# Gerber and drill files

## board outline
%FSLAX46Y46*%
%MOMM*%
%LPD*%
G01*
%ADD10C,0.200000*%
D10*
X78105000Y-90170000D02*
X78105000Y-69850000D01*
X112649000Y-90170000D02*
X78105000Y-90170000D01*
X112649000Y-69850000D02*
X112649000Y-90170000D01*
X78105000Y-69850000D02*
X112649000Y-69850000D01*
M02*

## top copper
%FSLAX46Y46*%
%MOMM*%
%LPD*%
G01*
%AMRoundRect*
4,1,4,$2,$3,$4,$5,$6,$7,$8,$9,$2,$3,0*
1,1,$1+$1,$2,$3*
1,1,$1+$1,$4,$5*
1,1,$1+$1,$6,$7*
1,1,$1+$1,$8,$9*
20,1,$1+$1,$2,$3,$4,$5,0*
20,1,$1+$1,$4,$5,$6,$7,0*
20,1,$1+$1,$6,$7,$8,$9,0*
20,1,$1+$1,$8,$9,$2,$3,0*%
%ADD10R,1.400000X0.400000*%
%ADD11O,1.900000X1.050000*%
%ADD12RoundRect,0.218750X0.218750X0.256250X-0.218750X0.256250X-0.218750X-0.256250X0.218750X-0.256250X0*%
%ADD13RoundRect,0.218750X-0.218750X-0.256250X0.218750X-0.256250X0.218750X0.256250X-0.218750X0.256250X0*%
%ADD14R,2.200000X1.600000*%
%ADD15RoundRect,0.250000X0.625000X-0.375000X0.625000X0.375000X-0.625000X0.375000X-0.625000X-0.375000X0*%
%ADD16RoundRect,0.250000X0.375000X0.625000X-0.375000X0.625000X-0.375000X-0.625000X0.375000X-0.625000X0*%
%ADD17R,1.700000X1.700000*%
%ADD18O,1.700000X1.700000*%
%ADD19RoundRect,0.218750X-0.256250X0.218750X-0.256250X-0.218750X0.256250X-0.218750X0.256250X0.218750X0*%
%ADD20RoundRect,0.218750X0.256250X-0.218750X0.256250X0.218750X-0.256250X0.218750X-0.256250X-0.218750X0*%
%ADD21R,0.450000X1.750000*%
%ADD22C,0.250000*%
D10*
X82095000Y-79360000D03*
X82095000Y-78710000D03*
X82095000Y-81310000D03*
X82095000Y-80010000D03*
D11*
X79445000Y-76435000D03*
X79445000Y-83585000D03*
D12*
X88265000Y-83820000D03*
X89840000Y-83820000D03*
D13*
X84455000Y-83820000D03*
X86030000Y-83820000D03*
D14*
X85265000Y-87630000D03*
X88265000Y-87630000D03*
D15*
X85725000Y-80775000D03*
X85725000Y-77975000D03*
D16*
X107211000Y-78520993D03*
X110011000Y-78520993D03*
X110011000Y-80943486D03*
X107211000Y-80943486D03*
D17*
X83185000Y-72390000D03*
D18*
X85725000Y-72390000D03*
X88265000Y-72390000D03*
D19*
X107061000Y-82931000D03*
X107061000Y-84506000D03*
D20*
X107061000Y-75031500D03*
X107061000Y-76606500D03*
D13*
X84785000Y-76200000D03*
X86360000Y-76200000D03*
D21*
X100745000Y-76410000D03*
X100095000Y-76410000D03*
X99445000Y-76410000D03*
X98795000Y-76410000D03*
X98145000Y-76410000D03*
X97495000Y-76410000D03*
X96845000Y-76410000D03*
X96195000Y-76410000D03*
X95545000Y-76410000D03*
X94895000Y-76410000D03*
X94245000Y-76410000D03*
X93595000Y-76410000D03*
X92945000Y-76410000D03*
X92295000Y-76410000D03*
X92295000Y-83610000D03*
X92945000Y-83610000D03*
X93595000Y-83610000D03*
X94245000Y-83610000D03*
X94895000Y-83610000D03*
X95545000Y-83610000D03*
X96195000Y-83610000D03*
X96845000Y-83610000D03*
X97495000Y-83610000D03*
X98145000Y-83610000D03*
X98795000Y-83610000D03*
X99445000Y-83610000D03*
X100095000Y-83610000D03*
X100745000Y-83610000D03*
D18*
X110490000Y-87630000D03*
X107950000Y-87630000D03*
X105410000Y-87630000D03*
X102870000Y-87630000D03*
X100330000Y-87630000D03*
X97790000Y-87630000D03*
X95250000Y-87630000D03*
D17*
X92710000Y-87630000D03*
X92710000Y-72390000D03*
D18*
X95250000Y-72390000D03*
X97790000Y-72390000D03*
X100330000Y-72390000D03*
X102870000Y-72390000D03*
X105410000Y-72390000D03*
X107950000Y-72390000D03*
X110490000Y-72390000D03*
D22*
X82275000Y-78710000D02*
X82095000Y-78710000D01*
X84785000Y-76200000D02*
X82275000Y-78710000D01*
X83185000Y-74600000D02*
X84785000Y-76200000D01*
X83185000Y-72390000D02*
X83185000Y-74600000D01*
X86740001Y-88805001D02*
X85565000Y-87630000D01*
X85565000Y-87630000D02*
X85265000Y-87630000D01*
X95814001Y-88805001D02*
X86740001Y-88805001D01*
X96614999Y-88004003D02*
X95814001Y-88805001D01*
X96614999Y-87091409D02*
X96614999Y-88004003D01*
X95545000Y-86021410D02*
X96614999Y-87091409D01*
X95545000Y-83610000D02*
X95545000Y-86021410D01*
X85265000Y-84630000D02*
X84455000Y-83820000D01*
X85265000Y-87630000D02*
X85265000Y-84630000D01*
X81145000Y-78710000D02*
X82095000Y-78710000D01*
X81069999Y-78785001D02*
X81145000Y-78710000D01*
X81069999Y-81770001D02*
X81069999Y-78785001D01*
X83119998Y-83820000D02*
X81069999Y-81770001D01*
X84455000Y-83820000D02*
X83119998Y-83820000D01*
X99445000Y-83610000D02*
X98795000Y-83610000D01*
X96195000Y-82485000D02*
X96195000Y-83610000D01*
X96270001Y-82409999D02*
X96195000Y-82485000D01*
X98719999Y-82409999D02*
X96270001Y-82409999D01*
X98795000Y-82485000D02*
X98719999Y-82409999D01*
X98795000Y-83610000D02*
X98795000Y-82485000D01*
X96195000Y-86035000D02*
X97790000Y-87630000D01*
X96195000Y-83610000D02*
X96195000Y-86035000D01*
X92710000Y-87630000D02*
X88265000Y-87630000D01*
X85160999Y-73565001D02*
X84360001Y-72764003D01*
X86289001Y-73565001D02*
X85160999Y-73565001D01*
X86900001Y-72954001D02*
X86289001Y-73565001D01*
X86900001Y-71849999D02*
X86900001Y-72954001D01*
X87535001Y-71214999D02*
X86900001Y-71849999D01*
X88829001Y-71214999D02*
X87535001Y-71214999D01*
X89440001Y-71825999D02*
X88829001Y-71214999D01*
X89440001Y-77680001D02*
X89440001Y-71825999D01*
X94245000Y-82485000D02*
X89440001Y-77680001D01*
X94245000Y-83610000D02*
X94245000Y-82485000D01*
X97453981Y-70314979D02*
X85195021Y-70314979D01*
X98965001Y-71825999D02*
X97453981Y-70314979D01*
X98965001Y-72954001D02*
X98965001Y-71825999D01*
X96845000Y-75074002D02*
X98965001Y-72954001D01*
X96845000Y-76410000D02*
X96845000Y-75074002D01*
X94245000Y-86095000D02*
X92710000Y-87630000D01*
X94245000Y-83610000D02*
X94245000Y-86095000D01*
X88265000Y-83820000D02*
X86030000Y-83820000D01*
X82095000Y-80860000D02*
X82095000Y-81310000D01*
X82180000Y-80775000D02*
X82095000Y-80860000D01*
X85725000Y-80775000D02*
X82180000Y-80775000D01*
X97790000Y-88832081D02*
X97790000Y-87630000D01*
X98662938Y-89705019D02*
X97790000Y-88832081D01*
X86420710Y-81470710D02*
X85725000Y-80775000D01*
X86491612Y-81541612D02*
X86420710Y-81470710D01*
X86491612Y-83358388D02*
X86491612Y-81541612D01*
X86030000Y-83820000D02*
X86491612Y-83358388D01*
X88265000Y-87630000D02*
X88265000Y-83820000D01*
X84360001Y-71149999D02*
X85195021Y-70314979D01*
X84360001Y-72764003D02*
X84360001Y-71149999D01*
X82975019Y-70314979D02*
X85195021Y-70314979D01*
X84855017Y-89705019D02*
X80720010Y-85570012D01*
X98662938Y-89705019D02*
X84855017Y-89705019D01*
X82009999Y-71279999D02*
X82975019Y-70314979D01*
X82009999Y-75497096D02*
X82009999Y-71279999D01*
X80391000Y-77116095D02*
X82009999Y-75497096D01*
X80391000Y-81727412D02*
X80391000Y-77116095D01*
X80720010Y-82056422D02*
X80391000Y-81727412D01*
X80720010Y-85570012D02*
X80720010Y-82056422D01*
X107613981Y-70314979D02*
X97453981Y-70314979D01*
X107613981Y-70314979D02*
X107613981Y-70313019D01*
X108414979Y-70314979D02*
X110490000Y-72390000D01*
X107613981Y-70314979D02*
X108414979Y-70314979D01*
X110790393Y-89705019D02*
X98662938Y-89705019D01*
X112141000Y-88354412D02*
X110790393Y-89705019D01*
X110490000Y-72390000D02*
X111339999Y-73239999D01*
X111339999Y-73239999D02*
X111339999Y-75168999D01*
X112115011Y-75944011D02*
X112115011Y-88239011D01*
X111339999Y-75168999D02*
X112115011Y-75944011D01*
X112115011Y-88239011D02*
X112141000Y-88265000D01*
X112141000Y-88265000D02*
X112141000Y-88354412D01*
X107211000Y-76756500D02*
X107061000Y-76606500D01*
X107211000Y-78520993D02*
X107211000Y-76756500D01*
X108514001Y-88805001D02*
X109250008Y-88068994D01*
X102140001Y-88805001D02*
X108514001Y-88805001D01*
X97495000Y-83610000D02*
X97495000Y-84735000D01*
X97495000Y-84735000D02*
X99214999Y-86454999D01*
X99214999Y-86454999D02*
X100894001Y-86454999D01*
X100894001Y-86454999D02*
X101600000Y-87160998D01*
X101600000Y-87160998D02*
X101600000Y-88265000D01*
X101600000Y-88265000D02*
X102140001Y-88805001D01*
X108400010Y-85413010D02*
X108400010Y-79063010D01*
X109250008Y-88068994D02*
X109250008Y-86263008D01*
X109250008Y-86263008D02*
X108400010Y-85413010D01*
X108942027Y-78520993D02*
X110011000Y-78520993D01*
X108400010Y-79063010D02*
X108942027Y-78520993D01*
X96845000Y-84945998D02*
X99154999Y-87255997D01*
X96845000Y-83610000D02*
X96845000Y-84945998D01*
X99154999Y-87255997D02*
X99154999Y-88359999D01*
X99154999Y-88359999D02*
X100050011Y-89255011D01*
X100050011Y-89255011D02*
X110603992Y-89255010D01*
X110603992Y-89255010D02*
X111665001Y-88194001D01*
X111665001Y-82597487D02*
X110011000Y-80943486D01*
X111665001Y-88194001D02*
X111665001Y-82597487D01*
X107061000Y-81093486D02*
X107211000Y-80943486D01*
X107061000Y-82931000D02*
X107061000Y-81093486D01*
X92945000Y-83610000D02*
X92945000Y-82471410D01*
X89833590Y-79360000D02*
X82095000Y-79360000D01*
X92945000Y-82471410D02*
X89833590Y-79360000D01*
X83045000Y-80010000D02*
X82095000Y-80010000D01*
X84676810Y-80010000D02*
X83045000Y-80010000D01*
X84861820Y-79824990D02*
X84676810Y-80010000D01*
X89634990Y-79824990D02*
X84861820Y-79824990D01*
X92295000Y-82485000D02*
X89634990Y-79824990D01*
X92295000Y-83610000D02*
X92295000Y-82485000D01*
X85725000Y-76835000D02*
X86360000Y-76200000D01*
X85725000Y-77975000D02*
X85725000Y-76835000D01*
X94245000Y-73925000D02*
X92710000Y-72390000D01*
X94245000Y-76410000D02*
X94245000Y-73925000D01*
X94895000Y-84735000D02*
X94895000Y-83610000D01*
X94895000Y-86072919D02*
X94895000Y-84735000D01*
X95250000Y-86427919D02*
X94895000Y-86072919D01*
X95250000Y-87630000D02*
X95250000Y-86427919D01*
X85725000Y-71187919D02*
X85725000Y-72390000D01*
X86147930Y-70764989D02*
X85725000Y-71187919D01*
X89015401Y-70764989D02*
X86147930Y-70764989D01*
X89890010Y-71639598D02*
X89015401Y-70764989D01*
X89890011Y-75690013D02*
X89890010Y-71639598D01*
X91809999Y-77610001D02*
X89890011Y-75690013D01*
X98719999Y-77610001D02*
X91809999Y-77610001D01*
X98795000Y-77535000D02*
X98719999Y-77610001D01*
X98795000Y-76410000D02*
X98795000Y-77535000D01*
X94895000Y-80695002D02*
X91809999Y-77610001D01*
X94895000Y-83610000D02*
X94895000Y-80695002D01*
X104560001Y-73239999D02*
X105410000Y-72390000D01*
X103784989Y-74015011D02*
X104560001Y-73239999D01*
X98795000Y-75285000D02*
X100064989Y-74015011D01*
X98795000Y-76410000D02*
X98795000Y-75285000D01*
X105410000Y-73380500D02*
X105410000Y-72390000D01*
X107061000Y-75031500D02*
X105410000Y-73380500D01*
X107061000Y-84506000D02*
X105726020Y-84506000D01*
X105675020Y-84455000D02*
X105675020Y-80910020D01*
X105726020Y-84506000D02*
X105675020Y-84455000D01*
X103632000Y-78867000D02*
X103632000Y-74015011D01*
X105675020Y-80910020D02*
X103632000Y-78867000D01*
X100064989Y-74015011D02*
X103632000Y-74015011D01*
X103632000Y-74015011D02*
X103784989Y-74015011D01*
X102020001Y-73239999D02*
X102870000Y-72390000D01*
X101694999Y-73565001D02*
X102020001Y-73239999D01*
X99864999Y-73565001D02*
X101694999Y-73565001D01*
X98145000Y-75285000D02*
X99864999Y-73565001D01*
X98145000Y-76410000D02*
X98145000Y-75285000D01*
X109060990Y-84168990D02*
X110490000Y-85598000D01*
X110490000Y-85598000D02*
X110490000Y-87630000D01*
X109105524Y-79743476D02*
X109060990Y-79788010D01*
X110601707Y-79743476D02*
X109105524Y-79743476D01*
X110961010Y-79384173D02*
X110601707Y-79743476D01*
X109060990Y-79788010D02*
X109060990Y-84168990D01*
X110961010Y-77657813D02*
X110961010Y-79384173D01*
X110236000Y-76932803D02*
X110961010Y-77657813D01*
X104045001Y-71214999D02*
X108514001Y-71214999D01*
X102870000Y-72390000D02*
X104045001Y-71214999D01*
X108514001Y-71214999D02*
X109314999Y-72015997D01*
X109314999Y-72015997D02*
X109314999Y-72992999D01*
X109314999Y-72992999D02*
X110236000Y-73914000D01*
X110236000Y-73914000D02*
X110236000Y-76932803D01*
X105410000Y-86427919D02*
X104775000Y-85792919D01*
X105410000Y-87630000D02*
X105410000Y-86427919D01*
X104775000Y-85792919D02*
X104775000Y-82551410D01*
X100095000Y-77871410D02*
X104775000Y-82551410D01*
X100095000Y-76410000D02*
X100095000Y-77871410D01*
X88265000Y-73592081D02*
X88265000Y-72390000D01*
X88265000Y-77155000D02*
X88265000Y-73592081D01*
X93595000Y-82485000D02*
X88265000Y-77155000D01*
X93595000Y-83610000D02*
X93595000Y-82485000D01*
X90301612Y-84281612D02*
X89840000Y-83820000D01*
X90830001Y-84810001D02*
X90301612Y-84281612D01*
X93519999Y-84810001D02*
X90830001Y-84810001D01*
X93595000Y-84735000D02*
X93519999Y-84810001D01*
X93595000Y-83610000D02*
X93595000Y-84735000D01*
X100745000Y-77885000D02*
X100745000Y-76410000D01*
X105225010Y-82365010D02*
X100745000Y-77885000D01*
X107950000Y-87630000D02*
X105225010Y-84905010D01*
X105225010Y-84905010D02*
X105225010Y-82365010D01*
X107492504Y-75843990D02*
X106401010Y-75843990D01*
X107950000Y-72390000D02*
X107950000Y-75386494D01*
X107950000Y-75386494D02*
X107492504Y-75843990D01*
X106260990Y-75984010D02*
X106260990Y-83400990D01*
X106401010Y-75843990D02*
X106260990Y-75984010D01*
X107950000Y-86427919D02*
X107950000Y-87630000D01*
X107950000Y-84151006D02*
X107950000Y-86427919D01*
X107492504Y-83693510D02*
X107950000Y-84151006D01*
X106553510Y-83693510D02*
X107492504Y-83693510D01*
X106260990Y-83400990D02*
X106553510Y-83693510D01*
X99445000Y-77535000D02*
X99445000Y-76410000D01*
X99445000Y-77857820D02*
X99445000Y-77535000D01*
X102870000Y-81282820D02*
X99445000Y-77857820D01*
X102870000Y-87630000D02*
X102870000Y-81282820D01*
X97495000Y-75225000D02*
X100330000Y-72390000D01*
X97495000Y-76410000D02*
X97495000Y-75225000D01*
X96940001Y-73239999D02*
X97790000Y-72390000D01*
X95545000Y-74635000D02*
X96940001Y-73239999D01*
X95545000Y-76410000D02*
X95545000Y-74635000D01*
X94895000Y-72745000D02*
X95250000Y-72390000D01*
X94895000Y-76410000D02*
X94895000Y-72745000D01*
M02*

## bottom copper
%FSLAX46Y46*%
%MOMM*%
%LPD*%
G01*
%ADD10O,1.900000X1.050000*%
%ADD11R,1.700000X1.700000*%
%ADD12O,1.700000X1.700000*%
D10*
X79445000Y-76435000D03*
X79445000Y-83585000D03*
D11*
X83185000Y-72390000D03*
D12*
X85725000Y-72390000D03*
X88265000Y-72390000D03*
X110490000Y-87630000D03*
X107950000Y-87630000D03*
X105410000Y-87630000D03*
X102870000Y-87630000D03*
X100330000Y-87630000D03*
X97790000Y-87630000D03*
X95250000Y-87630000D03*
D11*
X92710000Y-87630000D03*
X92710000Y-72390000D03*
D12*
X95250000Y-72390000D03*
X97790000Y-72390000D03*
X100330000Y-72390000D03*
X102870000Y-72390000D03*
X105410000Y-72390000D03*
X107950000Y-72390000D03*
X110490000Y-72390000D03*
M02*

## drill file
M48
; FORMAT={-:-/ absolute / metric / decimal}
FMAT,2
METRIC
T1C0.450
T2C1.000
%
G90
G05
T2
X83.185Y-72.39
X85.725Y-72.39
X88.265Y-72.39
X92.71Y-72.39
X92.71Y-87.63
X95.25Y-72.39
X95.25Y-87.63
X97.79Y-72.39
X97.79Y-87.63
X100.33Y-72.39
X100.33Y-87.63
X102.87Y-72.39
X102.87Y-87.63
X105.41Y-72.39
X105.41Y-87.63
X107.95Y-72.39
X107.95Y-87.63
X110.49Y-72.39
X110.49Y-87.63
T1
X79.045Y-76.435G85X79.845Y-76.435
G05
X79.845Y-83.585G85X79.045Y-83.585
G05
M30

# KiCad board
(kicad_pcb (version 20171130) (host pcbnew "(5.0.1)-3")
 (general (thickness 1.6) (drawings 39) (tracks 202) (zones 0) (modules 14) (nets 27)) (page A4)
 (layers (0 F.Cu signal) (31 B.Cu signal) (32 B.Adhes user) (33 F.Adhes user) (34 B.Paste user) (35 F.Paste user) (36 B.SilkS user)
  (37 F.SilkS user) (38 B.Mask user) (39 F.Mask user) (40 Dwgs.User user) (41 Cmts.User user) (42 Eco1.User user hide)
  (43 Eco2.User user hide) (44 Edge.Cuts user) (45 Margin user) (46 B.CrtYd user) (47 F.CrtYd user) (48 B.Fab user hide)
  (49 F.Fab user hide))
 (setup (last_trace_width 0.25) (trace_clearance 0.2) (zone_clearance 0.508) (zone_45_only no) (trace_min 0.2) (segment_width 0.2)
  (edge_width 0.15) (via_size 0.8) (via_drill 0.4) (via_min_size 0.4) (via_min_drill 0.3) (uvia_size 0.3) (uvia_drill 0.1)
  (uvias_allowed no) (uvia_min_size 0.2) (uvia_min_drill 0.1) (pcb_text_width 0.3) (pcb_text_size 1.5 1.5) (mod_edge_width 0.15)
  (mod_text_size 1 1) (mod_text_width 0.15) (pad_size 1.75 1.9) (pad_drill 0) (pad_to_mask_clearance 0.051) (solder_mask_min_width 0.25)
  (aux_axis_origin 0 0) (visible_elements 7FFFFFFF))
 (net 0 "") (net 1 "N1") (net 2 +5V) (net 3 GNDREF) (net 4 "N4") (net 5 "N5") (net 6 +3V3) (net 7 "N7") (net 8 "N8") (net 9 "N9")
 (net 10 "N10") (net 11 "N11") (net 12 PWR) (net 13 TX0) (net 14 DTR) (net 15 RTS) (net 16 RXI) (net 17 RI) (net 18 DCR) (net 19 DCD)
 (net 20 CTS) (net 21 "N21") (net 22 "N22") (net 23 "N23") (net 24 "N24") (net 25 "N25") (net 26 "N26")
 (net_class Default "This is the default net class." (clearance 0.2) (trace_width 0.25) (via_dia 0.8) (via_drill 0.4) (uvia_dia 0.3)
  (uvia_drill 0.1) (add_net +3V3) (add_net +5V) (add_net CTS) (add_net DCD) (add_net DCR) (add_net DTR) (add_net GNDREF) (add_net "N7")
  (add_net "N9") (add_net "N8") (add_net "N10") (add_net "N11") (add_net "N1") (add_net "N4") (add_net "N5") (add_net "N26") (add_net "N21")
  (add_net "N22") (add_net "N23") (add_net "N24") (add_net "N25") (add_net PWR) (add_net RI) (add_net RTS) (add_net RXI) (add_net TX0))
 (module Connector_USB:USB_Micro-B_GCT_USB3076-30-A (layer F.Cu) (at 80.645 80.01 270)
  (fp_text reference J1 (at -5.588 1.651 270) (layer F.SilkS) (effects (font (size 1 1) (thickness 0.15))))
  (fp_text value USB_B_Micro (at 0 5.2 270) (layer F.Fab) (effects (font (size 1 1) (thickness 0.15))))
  (pad 2 smd rect (at -0.65 -1.45 270) (size 0.4 1.4) (layers F.Cu F.Paste F.Mask) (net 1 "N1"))
  (pad 1 smd rect (at -1.3 -1.45 270) (size 0.4 1.4) (layers F.Cu F.Paste F.Mask) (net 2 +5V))
  (pad 5 smd rect (at 1.3 -1.45 270) (size 0.4 1.4) (layers F.Cu F.Paste F.Mask) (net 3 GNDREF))
  (pad 3 smd rect (at 0 -1.45 270) (size 0.4 1.4) (layers F.Cu F.Paste F.Mask) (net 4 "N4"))
  (pad 6 thru_hole oval (at -3.575 1.2 90) (size 1.05 1.9) (drill oval 0.45 1.25) (layers *.Cu *.Mask) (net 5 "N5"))
  (pad 6 thru_hole oval (at 3.575 1.2 270) (size 1.05 1.9) (drill oval 0.45 1.25) (layers *.Cu *.Mask) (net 5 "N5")))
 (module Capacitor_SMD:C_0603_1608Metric (layer F.Cu) (at 89.0525 83.82 180)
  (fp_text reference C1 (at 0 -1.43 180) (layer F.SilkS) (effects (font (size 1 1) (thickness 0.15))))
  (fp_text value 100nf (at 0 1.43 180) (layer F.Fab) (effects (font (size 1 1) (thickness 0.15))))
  (pad 2 smd roundrect (at 0.7875 0 180) (size 0.875 0.95) (layers F.Cu F.Paste F.Mask) (roundrect_rratio 0.25) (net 3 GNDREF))
  (pad 1 smd roundrect (at -0.7875 0 180) (size 0.875 0.95) (layers F.Cu F.Paste F.Mask) (roundrect_rratio 0.25) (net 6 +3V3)))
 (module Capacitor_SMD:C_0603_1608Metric (layer F.Cu) (at 85.2425 83.82)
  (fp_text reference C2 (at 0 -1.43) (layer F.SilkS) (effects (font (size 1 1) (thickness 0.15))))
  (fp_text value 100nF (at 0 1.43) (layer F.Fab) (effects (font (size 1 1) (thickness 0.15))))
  (pad 1 smd roundrect (at -0.7875 0) (size 0.875 0.95) (layers F.Cu F.Paste F.Mask) (roundrect_rratio 0.25) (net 2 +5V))
  (pad 2 smd roundrect (at 0.7875 0) (size 0.875 0.95) (layers F.Cu F.Paste F.Mask) (roundrect_rratio 0.25) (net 3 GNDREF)))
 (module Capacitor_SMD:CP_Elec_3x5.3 (layer F.Cu) (at 86.765 87.63)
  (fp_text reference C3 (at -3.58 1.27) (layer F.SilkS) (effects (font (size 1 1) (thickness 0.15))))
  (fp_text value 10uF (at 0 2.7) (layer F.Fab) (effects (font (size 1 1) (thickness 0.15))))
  (pad 1 smd rect (at -1.5 0) (size 2.2 1.6) (layers F.Cu F.Paste F.Mask) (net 2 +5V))
  (pad 2 smd rect (at 1.5 0) (size 2.2 1.6) (layers F.Cu F.Paste F.Mask) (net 3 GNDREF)))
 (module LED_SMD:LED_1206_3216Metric (layer F.Cu) (at 85.725 79.375 90)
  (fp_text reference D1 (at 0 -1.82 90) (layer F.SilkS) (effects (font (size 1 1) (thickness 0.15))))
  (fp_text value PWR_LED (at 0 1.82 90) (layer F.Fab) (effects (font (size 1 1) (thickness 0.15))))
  (pad 1 smd roundrect (at -1.4 0 90) (size 1.25 1.75) (layers F.Cu F.Paste F.Mask) (roundrect_rratio 0.2) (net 3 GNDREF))
  (pad 2 smd roundrect (at 1.4 0 90) (size 1.25 1.75) (layers F.Cu F.Paste F.Mask) (roundrect_rratio 0.2) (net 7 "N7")))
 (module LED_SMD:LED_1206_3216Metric (layer F.Cu) (at 108.611 78.520993 180)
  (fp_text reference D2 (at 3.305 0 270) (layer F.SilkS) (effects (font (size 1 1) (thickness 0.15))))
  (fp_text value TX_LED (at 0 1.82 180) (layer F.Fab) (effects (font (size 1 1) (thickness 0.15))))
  (pad 2 smd roundrect (at 1.4 0 180) (size 1.25 1.75) (layers F.Cu F.Paste F.Mask) (roundrect_rratio 0.2) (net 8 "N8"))
  (pad 1 smd roundrect (at -1.4 0 180) (size 1.25 1.75) (layers F.Cu F.Paste F.Mask) (roundrect_rratio 0.2) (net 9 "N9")))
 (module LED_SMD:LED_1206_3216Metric (layer F.Cu) (at 108.611 80.943486 180)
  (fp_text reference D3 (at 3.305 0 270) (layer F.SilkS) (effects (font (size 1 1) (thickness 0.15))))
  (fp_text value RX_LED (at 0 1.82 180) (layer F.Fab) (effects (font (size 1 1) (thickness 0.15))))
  (pad 1 smd roundrect (at -1.4 0 180) (size 1.25 1.75) (layers F.Cu F.Paste F.Mask) (roundrect_rratio 0.2) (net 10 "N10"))
  (pad 2 smd roundrect (at 1.4 0 180) (size 1.25 1.75) (layers F.Cu F.Paste F.Mask) (roundrect_rratio 0.2) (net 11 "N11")))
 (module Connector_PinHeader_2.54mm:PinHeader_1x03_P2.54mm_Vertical (layer F.Cu) (at 83.185 72.39 90)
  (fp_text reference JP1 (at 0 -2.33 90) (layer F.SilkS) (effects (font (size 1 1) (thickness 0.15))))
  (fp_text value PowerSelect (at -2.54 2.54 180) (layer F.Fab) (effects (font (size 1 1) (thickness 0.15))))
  (pad 1 thru_hole rect (at 0 0 90) (size 1.7 1.7) (drill 1) (layers *.Cu *.Mask) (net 2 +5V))
  (pad 2 thru_hole oval (at 0 2.54 90) (size 1.7 1.7) (drill 1) (layers *.Cu *.Mask) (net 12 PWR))
  (pad 3 thru_hole oval (at 0 5.08 90) (size 1.7 1.7) (drill 1) (layers *.Cu *.Mask) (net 6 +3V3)))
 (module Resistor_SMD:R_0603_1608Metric (layer F.Cu) (at 107.061 83.7185 270)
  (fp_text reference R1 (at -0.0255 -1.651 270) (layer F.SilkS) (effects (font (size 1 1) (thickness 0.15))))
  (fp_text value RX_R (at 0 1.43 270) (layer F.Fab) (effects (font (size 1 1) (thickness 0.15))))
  (pad 1 smd roundrect (at -0.7875 0 270) (size 0.875 0.95) (layers F.Cu F.Paste F.Mask) (roundrect_rratio 0.25) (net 11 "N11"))
  (pad 2 smd roundrect (at 0.7875 0 270) (size 0.875 0.95) (layers F.Cu F.Paste F.Mask) (roundrect_rratio 0.25) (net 12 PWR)))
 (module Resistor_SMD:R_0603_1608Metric (layer F.Cu) (at 107.061 75.819 90)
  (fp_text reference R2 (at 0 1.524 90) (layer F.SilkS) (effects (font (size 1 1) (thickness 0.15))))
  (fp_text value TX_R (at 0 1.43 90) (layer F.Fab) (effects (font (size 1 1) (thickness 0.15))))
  (pad 2 smd roundrect (at 0.7875 0 90) (size 0.875 0.95) (layers F.Cu F.Paste F.Mask) (roundrect_rratio 0.25) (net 12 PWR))
  (pad 1 smd roundrect (at -0.7875 0 90) (size 0.875 0.95) (layers F.Cu F.Paste F.Mask) (roundrect_rratio 0.25) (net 8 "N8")))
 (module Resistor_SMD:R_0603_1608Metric (layer F.Cu) (at 85.5725 76.2)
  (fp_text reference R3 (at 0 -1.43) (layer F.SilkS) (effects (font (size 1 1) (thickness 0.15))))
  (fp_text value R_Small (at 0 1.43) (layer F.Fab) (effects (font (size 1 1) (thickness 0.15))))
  (pad 1 smd roundrect (at -0.7875 0) (size 0.875 0.95) (layers F.Cu F.Paste F.Mask) (roundrect_rratio 0.25) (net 2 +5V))
  (pad 2 smd roundrect (at 0.7875 0) (size 0.875 0.95) (layers F.Cu F.Paste F.Mask) (roundrect_rratio 0.25) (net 7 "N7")))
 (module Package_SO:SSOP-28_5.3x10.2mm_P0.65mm (layer F.Cu) (at 96.52 80.01 270)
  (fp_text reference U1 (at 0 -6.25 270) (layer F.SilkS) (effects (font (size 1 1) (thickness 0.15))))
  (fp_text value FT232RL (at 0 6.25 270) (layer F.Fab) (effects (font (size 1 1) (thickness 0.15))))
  (pad 1 smd rect (at -3.6 -4.225 270) (size 1.75 0.45) (layers F.Cu F.Paste F.Mask) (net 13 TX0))
  (pad 2 smd rect (at -3.6 -3.575 270) (size 1.75 0.45) (layers F.Cu F.Paste F.Mask) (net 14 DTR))
  (pad 3 smd rect (at -3.6 -2.925 270) (size 1.75 0.45) (layers F.Cu F.Paste F.Mask) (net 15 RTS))
  (pad 4 smd rect (at -3.6 -2.275 270) (size 1.75 0.45) (layers F.Cu F.Paste F.Mask) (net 12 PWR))
  (pad 5 smd rect (at -3.6 -1.625 270) (size 1.75 0.45) (layers F.Cu F.Paste F.Mask) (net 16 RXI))
  (pad 6 smd rect (at -3.6 -0.975 270) (size 1.75 0.45) (layers F.Cu F.Paste F.Mask) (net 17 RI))
  (pad 7 smd rect (at -3.6 -0.325 270) (size 1.75 0.45) (layers F.Cu F.Paste F.Mask) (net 3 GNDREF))
  (pad 8 smd rect (at -3.6 0.325 270) (size 1.75 0.45) (layers F.Cu F.Paste F.Mask))
  (pad 9 smd rect (at -3.6 0.975 270) (size 1.75 0.45) (layers F.Cu F.Paste F.Mask) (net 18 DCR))
  (pad 10 smd rect (at -3.6 1.625 270) (size 1.75 0.45) (layers F.Cu F.Paste F.Mask) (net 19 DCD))
  (pad 11 smd rect (at -3.6 2.275 270) (size 1.75 0.45) (layers F.Cu F.Paste F.Mask) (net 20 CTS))
  (pad 12 smd rect (at -3.6 2.925 270) (size 1.75 0.45) (layers F.Cu F.Paste F.Mask) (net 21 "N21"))
  (pad 13 smd rect (at -3.6 3.575 270) (size 1.75 0.45) (layers F.Cu F.Paste F.Mask) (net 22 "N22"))
  (pad 14 smd rect (at -3.6 4.225 270) (size 1.75 0.45) (layers F.Cu F.Paste F.Mask) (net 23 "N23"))
  (pad 15 smd rect (at 3.6 4.225 270) (size 1.75 0.45) (layers F.Cu F.Paste F.Mask) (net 4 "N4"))
  (pad 16 smd rect (at 3.6 3.575 270) (size 1.75 0.45) (layers F.Cu F.Paste F.Mask) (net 1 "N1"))
  (pad 17 smd rect (at 3.6 2.925 270) (size 1.75 0.45) (layers F.Cu F.Paste F.Mask) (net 6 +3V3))
  (pad 18 smd rect (at 3.6 2.275 270) (size 1.75 0.45) (layers F.Cu F.Paste F.Mask) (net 3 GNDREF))
  (pad 19 smd rect (at 3.6 1.625 270) (size 1.75 0.45) (layers F.Cu F.Paste F.Mask) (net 12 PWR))
  (pad 20 smd rect (at 3.6 0.975 270) (size 1.75 0.45) (layers F.Cu F.Paste F.Mask) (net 2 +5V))
  (pad 21 smd rect (at 3.6 0.325 270) (size 1.75 0.45) (layers F.Cu F.Paste F.Mask) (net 3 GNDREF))
  (pad 22 smd rect (at 3.6 -0.325 270) (size 1.75 0.45) (layers F.Cu F.Paste F.Mask) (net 10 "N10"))
  (pad 23 smd rect (at 3.6 -0.975 270) (size 1.75 0.45) (layers F.Cu F.Paste F.Mask) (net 9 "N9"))
  (pad 24 smd rect (at 3.6 -1.625 270) (size 1.75 0.45) (layers F.Cu F.Paste F.Mask))
  (pad 25 smd rect (at 3.6 -2.275 270) (size 1.75 0.45) (layers F.Cu F.Paste F.Mask) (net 3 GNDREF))
  (pad 26 smd rect (at 3.6 -2.925 270) (size 1.75 0.45) (layers F.Cu F.Paste F.Mask) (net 3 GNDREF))
  (pad 27 smd rect (at 3.6 -3.575 270) (size 1.75 0.45) (layers F.Cu F.Paste F.Mask) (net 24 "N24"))
  (pad 28 smd rect (at 3.6 -4.225 270) (size 1.75 0.45) (layers F.Cu F.Paste F.Mask) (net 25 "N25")))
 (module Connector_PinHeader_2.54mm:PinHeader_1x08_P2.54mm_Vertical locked (layer F.Cu) (at 92.71 87.63 90)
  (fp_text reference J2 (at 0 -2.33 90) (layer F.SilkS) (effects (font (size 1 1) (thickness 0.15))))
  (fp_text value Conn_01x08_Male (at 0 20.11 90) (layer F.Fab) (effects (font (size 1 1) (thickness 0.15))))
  (pad 8 thru_hole oval (at 0 17.78 90) (size 1.7 1.7) (drill 1) (layers *.Cu *.Mask) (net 16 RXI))
  (pad 7 thru_hole oval (at 0 15.24 90) (size 1.7 1.7) (drill 1) (layers *.Cu *.Mask) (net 13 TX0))
  (pad 6 thru_hole oval (at 0 12.7 90) (size 1.7 1.7) (drill 1) (layers *.Cu *.Mask) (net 14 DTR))
  (pad 5 thru_hole oval (at 0 10.16 90) (size 1.7 1.7) (drill 1) (layers *.Cu *.Mask) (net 15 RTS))
  (pad 4 thru_hole oval (at 0 7.62 90) (size 1.7 1.7) (drill 1) (layers *.Cu *.Mask) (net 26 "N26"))
  (pad 3 thru_hole oval (at 0 5.08 90) (size 1.7 1.7) (drill 1) (layers *.Cu *.Mask) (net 3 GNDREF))
  (pad 2 thru_hole oval (at 0 2.54 90) (size 1.7 1.7) (drill 1) (layers *.Cu *.Mask) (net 12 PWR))
  (pad 1 thru_hole rect (at 0 0 90) (size 1.7 1.7) (drill 1) (layers *.Cu *.Mask) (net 3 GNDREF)))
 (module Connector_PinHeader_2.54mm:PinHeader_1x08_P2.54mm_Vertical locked (layer F.Cu) (at 92.71 72.39 90)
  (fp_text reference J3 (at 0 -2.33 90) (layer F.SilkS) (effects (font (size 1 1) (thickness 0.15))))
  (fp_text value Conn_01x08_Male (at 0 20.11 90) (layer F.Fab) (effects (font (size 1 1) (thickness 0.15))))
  (pad 1 thru_hole rect (at 0 0 90) (size 1.7 1.7) (drill 1) (layers *.Cu *.Mask) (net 20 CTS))
  (pad 2 thru_hole oval (at 0 2.54 90) (size 1.7 1.7) (drill 1) (layers *.Cu *.Mask) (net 19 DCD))
  (pad 3 thru_hole oval (at 0 5.08 90) (size 1.7 1.7) (drill 1) (layers *.Cu *.Mask) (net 18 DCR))
  (pad 4 thru_hole oval (at 0 7.62 90) (size 1.7 1.7) (drill 1) (layers *.Cu *.Mask) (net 17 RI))
  (pad 5 thru_hole oval (at 0 10.16 90) (size 1.7 1.7) (drill 1) (layers *.Cu *.Mask) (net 16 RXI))
  (pad 6 thru_hole oval (at 0 12.7 90) (size 1.7 1.7) (drill 1) (layers *.Cu *.Mask) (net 12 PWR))
  (pad 7 thru_hole oval (at 0 15.24 90) (size 1.7 1.7) (drill 1) (layers *.Cu *.Mask) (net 13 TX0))
  (pad 8 thru_hole oval (at 0 17.78 90) (size 1.7 1.7) (drill 1) (layers *.Cu *.Mask) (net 3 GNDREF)))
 (gr_line (start 78.105 90.17) (end 78.105 69.85) (layer Edge.Cuts) (width 0.2))
 (gr_line (start 112.649 90.17) (end 78.105 90.17) (layer Edge.Cuts) (width 0.2))
 (gr_line (start 112.649 69.85) (end 112.649 90.17) (layer Edge.Cuts) (width 0.2))
 (gr_line (start 78.105 69.85) (end 112.649 69.85) (layer Edge.Cuts) (width 0.2))
 (segment (start 82.275 78.71) (end 82.095 78.71) (width 0.25) (layer F.Cu) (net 2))
 (segment (start 84.785 76.2) (end 82.275 78.71) (width 0.25) (layer F.Cu) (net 2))
 (segment (start 83.185 74.6) (end 84.785 76.2) (width 0.25) (layer F.Cu) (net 2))
 (segment (start 83.185 72.39) (end 83.185 74.6) (width 0.25) (layer F.Cu) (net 2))
 (segment (start 86.740001 88.805001) (end 85.565 87.63) (width 0.25) (layer F.Cu) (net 2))
 (segment (start 85.565 87.63) (end 85.265 87.63) (width 0.25) (layer F.Cu) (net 2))
 (segment (start 95.814001 88.805001) (end 86.740001 88.805001) (width 0.25) (layer F.Cu) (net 2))
 (segment (start 96.614999 88.004003) (end 95.814001 88.805001) (width 0.25) (layer F.Cu) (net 2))
 (segment (start 96.614999 87.091409) (end 96.614999 88.004003) (width 0.25) (layer F.Cu) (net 2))
 (segment (start 95.545 86.02141) (end 96.614999 87.091409) (width 0.25) (layer F.Cu) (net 2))
 (segment (start 95.545 83.61) (end 95.545 86.02141) (width 0.25) (layer F.Cu) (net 2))
 (segment (start 85.265 84.63) (end 84.455 83.82) (width 0.25) (layer F.Cu) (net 2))
 (segment (start 85.265 87.63) (end 85.265 84.63) (width 0.25) (layer F.Cu) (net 2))
 (segment (start 81.145 78.71) (end 82.095 78.71) (width 0.25) (layer F.Cu) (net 2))
 (segment (start 81.069999 78.785001) (end 81.145 78.71) (width 0.25) (layer F.Cu) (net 2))
 (segment (start 81.069999 81.770001) (end 81.069999 78.785001) (width 0.25) (layer F.Cu) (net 2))
 (segment (start 83.119998 83.82) (end 81.069999 81.770001) (width 0.25) (layer F.Cu) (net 2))
 (segment (start 84.455 83.82) (end 83.119998 83.82) (width 0.25) (layer F.Cu) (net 2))
 (segment (start 99.445 83.61) (end 98.795 83.61) (width 0.25) (layer F.Cu) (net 3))
 (segment (start 96.195 82.485) (end 96.195 83.61) (width 0.25) (layer F.Cu) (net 3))
 (segment (start 96.270001 82.409999) (end 96.195 82.485) (width 0.25) (layer F.Cu) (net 3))
 (segment (start 98.719999 82.409999) (end 96.270001 82.409999) (width 0.25) (layer F.Cu) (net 3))
 (segment (start 98.795 82.485) (end 98.719999 82.409999) (width 0.25) (layer F.Cu) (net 3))
 (segment (start 98.795 83.61) (end 98.795 82.485) (width 0.25) (layer F.Cu) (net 3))
 (segment (start 96.195 86.035) (end 97.79 87.63) (width 0.25) (layer F.Cu) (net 3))
 (segment (start 96.195 83.61) (end 96.195 86.035) (width 0.25) (layer F.Cu) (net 3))
 (segment (start 92.71 87.63) (end 88.265 87.63) (width 0.25) (layer F.Cu) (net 3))
 (segment (start 85.160999 73.565001) (end 84.360001 72.764003) (width 0.25) (layer F.Cu) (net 3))
 (segment (start 86.289001 73.565001) (end 85.160999 73.565001) (width 0.25) (layer F.Cu) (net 3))
 (segment (start 86.900001 72.954001) (end 86.289001 73.565001) (width 0.25) (layer F.Cu) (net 3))
 (segment (start 86.900001 71.849999) (end 86.900001 72.954001) (width 0.25) (layer F.Cu) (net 3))
 (segment (start 87.535001 71.214999) (end 86.900001 71.849999) (width 0.25) (layer F.Cu) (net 3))
 (segment (start 88.829001 71.214999) (end 87.535001 71.214999) (width 0.25) (layer F.Cu) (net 3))
 (segment (start 89.440001 71.825999) (end 88.829001 71.214999) (width 0.25) (layer F.Cu) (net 3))
 (segment (start 89.440001 77.680001) (end 89.440001 71.825999) (width 0.25) (layer F.Cu) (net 3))
 (segment (start 94.245 82.485) (end 89.440001 77.680001) (width 0.25) (layer F.Cu) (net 3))
 (segment (start 94.245 83.61) (end 94.245 82.485) (width 0.25) (layer F.Cu) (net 3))
 (segment (start 97.453981 70.314979) (end 85.195021 70.314979) (width 0.25) (layer F.Cu) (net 3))
 (segment (start 98.965001 71.825999) (end 97.453981 70.314979) (width 0.25) (layer F.Cu) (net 3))
 (segment (start 98.965001 72.954001) (end 98.965001 71.825999) (width 0.25) (layer F.Cu) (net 3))
 (segment (start 96.845 75.074002) (end 98.965001 72.954001) (width 0.25) (layer F.Cu) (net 3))
 (segment (start 96.845 76.41) (end 96.845 75.074002) (width 0.25) (layer F.Cu) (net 3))
 (segment (start 94.245 86.095) (end 92.71 87.63) (width 0.25) (layer F.Cu) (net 3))
 (segment (start 94.245 83.61) (end 94.245 86.095) (width 0.25) (layer F.Cu) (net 3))
 (segment (start 88.265 83.82) (end 86.03 83.82) (width 0.25) (layer F.Cu) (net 3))
 (segment (start 82.095 80.86) (end 82.095 81.31) (width 0.25) (layer F.Cu) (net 3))
 (segment (start 82.18 80.775) (end 82.095 80.86) (width 0.25) (layer F.Cu) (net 3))
 (segment (start 85.725 80.775) (end 82.18 80.775) (width 0.25) (layer F.Cu) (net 3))
 (segment (start 97.79 88.832081) (end 97.79 87.63) (width 0.25) (layer F.Cu) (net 3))
 (segment (start 98.662938 89.705019) (end 97.79 88.832081) (width 0.25) (layer F.Cu) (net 3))
 (segment (start 86.42071 81.47071) (end 85.725 80.775) (width 0.25) (layer F.Cu) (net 3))
 (segment (start 86.491612 81.541612) (end 86.42071 81.47071) (width 0.25) (layer F.Cu) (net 3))
 (segment (start 86.491612 83.358388) (end 86.491612 81.541612) (width 0.25) (layer F.Cu) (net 3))
 (segment (start 86.03 83.82) (end 86.491612 83.358388) (width 0.25) (layer F.Cu) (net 3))
 (segment (start 88.265 87.63) (end 88.265 83.82) (width 0.25) (layer F.Cu) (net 3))
 (segment (start 84.360001 71.149999) (end 85.195021 70.314979) (width 0.25) (layer F.Cu) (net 3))
 (segment (start 84.360001 72.764003) (end 84.360001 71.149999) (width 0.25) (layer F.Cu) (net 3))
 (segment (start 82.975019 70.314979) (end 85.195021 70.314979) (width 0.25) (layer F.Cu) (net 3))
 (segment (start 84.855017 89.705019) (end 80.72001 85.570012) (width 0.25) (layer F.Cu) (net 3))
 (segment (start 98.662938 89.705019) (end 84.855017 89.705019) (width 0.25) (layer F.Cu) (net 3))
 (segment (start 82.009999 71.279999) (end 82.975019 70.314979) (width 0.25) (layer F.Cu) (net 3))
 (segment (start 82.009999 75.497096) (end 82.009999 71.279999) (width 0.25) (layer F.Cu) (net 3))
 (segment (start 80.391 77.116095) (end 82.009999 75.497096) (width 0.25) (layer F.Cu) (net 3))
 (segment (start 80.391 81.727412) (end 80.391 77.116095) (width 0.25) (layer F.Cu) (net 3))
 (segment (start 80.72001 82.056422) (end 80.391 81.727412) (width 0.25) (layer F.Cu) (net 3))
 (segment (start 80.72001 85.570012) (end 80.72001 82.056422) (width 0.25) (layer F.Cu) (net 3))
 (segment (start 107.613981 70.314979) (end 97.453981 70.314979) (width 0.25) (layer F.Cu) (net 3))
 (segment (start 107.613981 70.314979) (end 107.613981 70.313019) (width 0.25) (layer F.Cu) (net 3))
 (segment (start 108.414979 70.314979) (end 110.49 72.39) (width 0.25) (layer F.Cu) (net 3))
 (segment (start 107.613981 70.314979) (end 108.414979 70.314979) (width 0.25) (layer F.Cu) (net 3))
 (segment (start 110.790393 89.705019) (end 98.662938 89.705019) (width 0.25) (layer F.Cu) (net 3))
 (segment (start 112.141 88.354412) (end 110.790393 89.705019) (width 0.25) (layer F.Cu) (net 3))
 (segment (start 110.49 72.39) (end 111.339999 73.239999) (width 0.25) (layer F.Cu) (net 3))
 (segment (start 111.339999 73.239999) (end 111.339999 75.168999) (width 0.25) (layer F.Cu) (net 3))
 (segment (start 112.115011 75.944011) (end 112.115011 88.239011) (width 0.25) (layer F.Cu) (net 3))
 (segment (start 111.339999 75.168999) (end 112.115011 75.944011) (width 0.25) (layer F.Cu) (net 3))
 (segment (start 112.115011 88.239011) (end 112.141 88.265) (width 0.25) (layer F.Cu) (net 3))
 (segment (start 112.141 88.265) (end 112.141 88.354412) (width 0.25) (layer F.Cu) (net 3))
 (segment (start 107.211 76.7565) (end 107.061 76.6065) (width 0.25) (layer F.Cu) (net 8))
 (segment (start 107.211 78.520993) (end 107.211 76.7565) (width 0.25) (layer F.Cu) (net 8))
 (segment (start 108.514001 88.805001) (end 109.250008 88.068994) (width 0.25) (layer F.Cu) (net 9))
 (segment (start 102.140001 88.805001) (end 108.514001 88.805001) (width 0.25) (layer F.Cu) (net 9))
 (segment (start 97.495 83.61) (end 97.495 84.735) (width 0.25) (layer F.Cu) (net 9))
 (segment (start 97.495 84.735) (end 99.214999 86.454999) (width 0.25) (layer F.Cu) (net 9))
 (segment (start 99.214999 86.454999) (end 100.894001 86.454999) (width 0.25) (layer F.Cu) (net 9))
 (segment (start 100.894001 86.454999) (end 101.6 87.160998) (width 0.25) (layer F.Cu) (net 9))
 (segment (start 101.6 87.160998) (end 101.6 88.265) (width 0.25) (layer F.Cu) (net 9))
 (segment (start 101.6 88.265) (end 102.140001 88.805001) (width 0.25) (layer F.Cu) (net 9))
 (segment (start 108.40001 85.41301) (end 108.40001 79.06301) (width 0.25) (layer F.Cu) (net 9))
 (segment (start 109.250008 88.068994) (end 109.250008 86.263008) (width 0.25) (layer F.Cu) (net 9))
 (segment (start 109.250008 86.263008) (end 108.40001 85.41301) (width 0.25) (layer F.Cu) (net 9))
 (segment (start 108.942027 78.520993) (end 110.011 78.520993) (width 0.25) (layer F.Cu) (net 9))
 (segment (start 108.40001 79.06301) (end 108.942027 78.520993) (width 0.25) (layer F.Cu) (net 9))
 (segment (start 96.845 84.945998) (end 99.154999 87.255997) (width 0.25) (layer F.Cu) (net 10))
 (segment (start 96.845 83.61) (end 96.845 84.945998) (width 0.25) (layer F.Cu) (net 10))
 (segment (start 99.154999 87.255997) (end 99.154999 88.359999) (width 0.25) (layer F.Cu) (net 10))
 (segment (start 99.154999 88.359999) (end 100.050011 89.255011) (width 0.25) (layer F.Cu) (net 10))
 (segment (start 100.050011 89.255011) (end 110.603992 89.25501) (width 0.25) (layer F.Cu) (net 10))
 (segment (start 110.603992 89.25501) (end 111.665001 88.194001) (width 0.25) (layer F.Cu) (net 10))
 (segment (start 111.665001 82.597487) (end 110.011 80.943486) (width 0.25) (layer F.Cu) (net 10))
 (segment (start 111.665001 88.194001) (end 111.665001 82.597487) (width 0.25) (layer F.Cu) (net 10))
 (segment (start 107.061 81.093486) (end 107.211 80.943486) (width 0.25) (layer F.Cu) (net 11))
 (segment (start 107.061 82.931) (end 107.061 81.093486) (width 0.25) (layer F.Cu) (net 11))
 (segment (start 92.945 83.61) (end 92.945 82.47141) (width 0.25) (layer F.Cu) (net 1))
 (segment (start 89.83359 79.36) (end 82.095 79.36) (width 0.25) (layer F.Cu) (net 1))
 (segment (start 92.945 82.47141) (end 89.83359 79.36) (width 0.25) (layer F.Cu) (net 1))
 (segment (start 83.045 80.01) (end 82.095 80.01) (width 0.25) (layer F.Cu) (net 4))
 (segment (start 84.67681 80.01) (end 83.045 80.01) (width 0.25) (layer F.Cu) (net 4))
 (segment (start 84.86182 79.82499) (end 84.67681 80.01) (width 0.25) (layer F.Cu) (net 4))
 (segment (start 89.63499 79.82499) (end 84.86182 79.82499) (width 0.25) (layer F.Cu) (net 4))
 (segment (start 92.295 82.485) (end 89.63499 79.82499) (width 0.25) (layer F.Cu) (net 4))
 (segment (start 92.295 83.61) (end 92.295 82.485) (width 0.25) (layer F.Cu) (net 4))
 (segment (start 85.725 76.835) (end 86.36 76.2) (width 0.25) (layer F.Cu) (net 7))
 (segment (start 85.725 77.975) (end 85.725 76.835) (width 0.25) (layer F.Cu) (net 7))
 (segment (start 94.245 73.925) (end 92.71 72.39) (width 0.25) (layer F.Cu) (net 20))
 (segment (start 94.245 76.41) (end 94.245 73.925) (width 0.25) (layer F.Cu) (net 20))
 (segment (start 94.895 84.735) (end 94.895 83.61) (width 0.25) (layer F.Cu) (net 12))
 (segment (start 94.895 86.072919) (end 94.895 84.735) (width 0.25) (layer F.Cu) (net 12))
 (segment (start 95.25 86.427919) (end 94.895 86.072919) (width 0.25) (layer F.Cu) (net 12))
 (segment (start 95.25 87.63) (end 95.25 86.427919) (width 0.25) (layer F.Cu) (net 12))
 (segment (start 85.725 71.187919) (end 85.725 72.39) (width 0.25) (layer F.Cu) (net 12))
 (segment (start 86.14793 70.764989) (end 85.725 71.187919) (width 0.25) (layer F.Cu) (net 12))
 (segment (start 89.015401 70.764989) (end 86.14793 70.764989) (width 0.25) (layer F.Cu) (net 12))
 (segment (start 89.89001 71.639598) (end 89.015401 70.764989) (width 0.25) (layer F.Cu) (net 12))
 (segment (start 89.890011 75.690013) (end 89.89001 71.639598) (width 0.25) (layer F.Cu) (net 12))
 (segment (start 91.809999 77.610001) (end 89.890011 75.690013) (width 0.25) (layer F.Cu) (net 12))
 (segment (start 98.719999 77.610001) (end 91.809999 77.610001) (width 0.25) (layer F.Cu) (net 12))
 (segment (start 98.795 77.535) (end 98.719999 77.610001) (width 0.25) (layer F.Cu) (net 12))
 (segment (start 98.795 76.41) (end 98.795 77.535) (width 0.25) (layer F.Cu) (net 12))
 (segment (start 94.895 80.695002) (end 91.809999 77.610001) (width 0.25) (layer F.Cu) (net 12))
 (segment (start 94.895 83.61) (end 94.895 80.695002) (width 0.25) (layer F.Cu) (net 12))
 (segment (start 104.560001 73.239999) (end 105.41 72.39) (width 0.25) (layer F.Cu) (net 12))
 (segment (start 103.784989 74.015011) (end 104.560001 73.239999) (width 0.25) (layer F.Cu) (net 12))
 (segment (start 98.795 75.285) (end 100.064989 74.015011) (width 0.25) (layer F.Cu) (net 12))
 (segment (start 98.795 76.41) (end 98.795 75.285) (width 0.25) (layer F.Cu) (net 12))
 (segment (start 105.41 73.3805) (end 105.41 72.39) (width 0.25) (layer F.Cu) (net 12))
 (segment (start 107.061 75.0315) (end 105.41 73.3805) (width 0.25) (layer F.Cu) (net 12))
 (segment (start 107.061 84.506) (end 105.72602 84.506) (width 0.25) (layer F.Cu) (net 12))
 (segment (start 105.67502 84.455) (end 105.67502 80.91002) (width 0.25) (layer F.Cu) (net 12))
 (segment (start 105.72602 84.506) (end 105.67502 84.455) (width 0.25) (layer F.Cu) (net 12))
 (segment (start 103.632 78.867) (end 103.632 74.015011) (width 0.25) (layer F.Cu) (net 12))
 (segment (start 105.67502 80.91002) (end 103.632 78.867) (width 0.25) (layer F.Cu) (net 12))
 (segment (start 100.064989 74.015011) (end 103.632 74.015011) (width 0.25) (layer F.Cu) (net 12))
 (segment (start 103.632 74.015011) (end 103.784989 74.015011) (width 0.25) (layer F.Cu) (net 12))
 (segment (start 102.020001 73.239999) (end 102.87 72.39) (width 0.25) (layer F.Cu) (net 16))
 (segment (start 101.694999 73.565001) (end 102.020001 73.239999) (width 0.25) (layer F.Cu) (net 16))
 (segment (start 99.864999 73.565001) (end 101.694999 73.565001) (width 0.25) (layer F.Cu) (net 16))
 (segment (start 98.145 75.285) (end 99.864999 73.565001) (width 0.25) (layer F.Cu) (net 16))
 (segment (start 98.145 76.41) (end 98.145 75.285) (width 0.25) (layer F.Cu) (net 16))
 (segment (start 109.06099 84.16899) (end 110.49 85.598) (width 0.25) (layer F.Cu) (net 16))
 (segment (start 110.49 85.598) (end 110.49 87.63) (width 0.25) (layer F.Cu) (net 16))
 (segment (start 109.105524 79.743476) (end 109.06099 79.78801) (width 0.25) (layer F.Cu) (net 16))
 (segment (start 110.601707 79.743476) (end 109.105524 79.743476) (width 0.25) (layer F.Cu) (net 16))
 (segment (start 110.96101 79.384173) (end 110.601707 79.743476) (width 0.25) (layer F.Cu) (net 16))
 (segment (start 109.06099 79.78801) (end 109.06099 84.16899) (width 0.25) (layer F.Cu) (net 16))
 (segment (start 110.96101 77.657813) (end 110.96101 79.384173) (width 0.25) (layer F.Cu) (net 16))
 (segment (start 110.236 76.932803) (end 110.96101 77.657813) (width 0.25) (layer F.Cu) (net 16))
 (segment (start 104.045001 71.214999) (end 108.514001 71.214999) (width 0.25) (layer F.Cu) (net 16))
 (segment (start 102.87 72.39) (end 104.045001 71.214999) (width 0.25) (layer F.Cu) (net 16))
 (segment (start 108.514001 71.214999) (end 109.314999 72.015997) (width 0.25) (layer F.Cu) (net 16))
 (segment (start 109.314999 72.015997) (end 109.314999 72.992999) (width 0.25) (layer F.Cu) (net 16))
 (segment (start 109.314999 72.992999) (end 110.236 73.914) (width 0.25) (layer F.Cu) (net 16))
 (segment (start 110.236 73.914) (end 110.236 76.932803) (width 0.25) (layer F.Cu) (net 16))
 (segment (start 105.41 86.427919) (end 104.775 85.792919) (width 0.25) (layer F.Cu) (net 14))
 (segment (start 105.41 87.63) (end 105.41 86.427919) (width 0.25) (layer F.Cu) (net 14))
 (segment (start 104.775 85.792919) (end 104.775 82.55141) (width 0.25) (layer F.Cu) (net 14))
 (segment (start 100.095 77.87141) (end 104.775 82.55141) (width 0.25) (layer F.Cu) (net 14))
 (segment (start 100.095 76.41) (end 100.095 77.87141) (width 0.25) (layer F.Cu) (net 14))
 (segment (start 88.265 73.592081) (end 88.265 72.39) (width 0.25) (layer F.Cu) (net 6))
 (segment (start 88.265 77.155) (end 88.265 73.592081) (width 0.25) (layer F.Cu) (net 6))
 (segment (start 93.595 82.485) (end 88.265 77.155) (width 0.25) (layer F.Cu) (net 6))
 (segment (start 93.595 83.61) (end 93.595 82.485) (width 0.25) (layer F.Cu) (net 6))
 (segment (start 90.301612 84.281612) (end 89.84 83.82) (width 0.25) (layer F.Cu) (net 6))
 (segment (start 90.830001 84.810001) (end 90.301612 84.281612) (width 0.25) (layer F.Cu) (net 6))
 (segment (start 93.519999 84.810001) (end 90.830001 84.810001) (width 0.25) (layer F.Cu) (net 6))
 (segment (start 93.595 84.735) (end 93.519999 84.810001) (width 0.25) (layer F.Cu) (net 6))
 (segment (start 93.595 83.61) (end 93.595 84.735) (width 0.25) (layer F.Cu) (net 6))
 (segment (start 100.745 77.885) (end 100.745 76.41) (width 0.25) (layer F.Cu) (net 13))
 (segment (start 105.22501 82.36501) (end 100.745 77.885) (width 0.25) (layer F.Cu) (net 13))
 (segment (start 107.95 87.63) (end 105.22501 84.90501) (width 0.25) (layer F.Cu) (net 13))
 (segment (start 105.22501 84.90501) (end 105.22501 82.36501) (width 0.25) (layer F.Cu) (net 13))
 (segment (start 107.492504 75.84399) (end 106.40101 75.84399) (width 0.25) (layer F.Cu) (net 13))
 (segment (start 107.95 72.39) (end 107.95 75.386494) (width 0.25) (layer F.Cu) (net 13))
 (segment (start 107.95 75.386494) (end 107.492504 75.84399) (width 0.25) (layer F.Cu) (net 13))
 (segment (start 106.26099 75.98401) (end 106.26099 83.40099) (width 0.25) (layer F.Cu) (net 13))
 (segment (start 106.40101 75.84399) (end 106.26099 75.98401) (width 0.25) (layer F.Cu) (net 13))
 (segment (start 107.95 86.427919) (end 107.95 87.63) (width 0.25) (layer F.Cu) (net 13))
 (segment (start 107.95 84.151006) (end 107.95 86.427919) (width 0.25) (layer F.Cu) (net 13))
 (segment (start 107.492504 83.69351) (end 107.95 84.151006) (width 0.25) (layer F.Cu) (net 13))
 (segment (start 106.55351 83.69351) (end 107.492504 83.69351) (width 0.25) (layer F.Cu) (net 13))
 (segment (start 106.26099 83.40099) (end 106.55351 83.69351) (width 0.25) (layer F.Cu) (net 13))
 (segment (start 99.445 77.535) (end 99.445 76.41) (width 0.25) (layer F.Cu) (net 15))
 (segment (start 99.445 77.85782) (end 99.445 77.535) (width 0.25) (layer F.Cu) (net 15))
 (segment (start 102.87 81.28282) (end 99.445 77.85782) (width 0.25) (layer F.Cu) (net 15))
 (segment (start 102.87 87.63) (end 102.87 81.28282) (width 0.25) (layer F.Cu) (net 15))
 (segment (start 97.495 75.225) (end 100.33 72.39) (width 0.25) (layer F.Cu) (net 17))
 (segment (start 97.495 76.41) (end 97.495 75.225) (width 0.25) (layer F.Cu) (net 17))
 (segment (start 96.940001 73.239999) (end 97.79 72.39) (width 0.25) (layer F.Cu) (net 18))
 (segment (start 95.545 74.635) (end 96.940001 73.239999) (width 0.25) (layer F.Cu) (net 18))
 (segment (start 95.545 76.41) (end 95.545 74.635) (width 0.25) (layer F.Cu) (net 18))
 (segment (start 94.895 72.745) (end 95.25 72.39) (width 0.25) (layer F.Cu) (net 19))
 (segment (start 94.895 76.41) (end 94.895 72.745) (width 0.25) (layer F.Cu) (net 19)))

